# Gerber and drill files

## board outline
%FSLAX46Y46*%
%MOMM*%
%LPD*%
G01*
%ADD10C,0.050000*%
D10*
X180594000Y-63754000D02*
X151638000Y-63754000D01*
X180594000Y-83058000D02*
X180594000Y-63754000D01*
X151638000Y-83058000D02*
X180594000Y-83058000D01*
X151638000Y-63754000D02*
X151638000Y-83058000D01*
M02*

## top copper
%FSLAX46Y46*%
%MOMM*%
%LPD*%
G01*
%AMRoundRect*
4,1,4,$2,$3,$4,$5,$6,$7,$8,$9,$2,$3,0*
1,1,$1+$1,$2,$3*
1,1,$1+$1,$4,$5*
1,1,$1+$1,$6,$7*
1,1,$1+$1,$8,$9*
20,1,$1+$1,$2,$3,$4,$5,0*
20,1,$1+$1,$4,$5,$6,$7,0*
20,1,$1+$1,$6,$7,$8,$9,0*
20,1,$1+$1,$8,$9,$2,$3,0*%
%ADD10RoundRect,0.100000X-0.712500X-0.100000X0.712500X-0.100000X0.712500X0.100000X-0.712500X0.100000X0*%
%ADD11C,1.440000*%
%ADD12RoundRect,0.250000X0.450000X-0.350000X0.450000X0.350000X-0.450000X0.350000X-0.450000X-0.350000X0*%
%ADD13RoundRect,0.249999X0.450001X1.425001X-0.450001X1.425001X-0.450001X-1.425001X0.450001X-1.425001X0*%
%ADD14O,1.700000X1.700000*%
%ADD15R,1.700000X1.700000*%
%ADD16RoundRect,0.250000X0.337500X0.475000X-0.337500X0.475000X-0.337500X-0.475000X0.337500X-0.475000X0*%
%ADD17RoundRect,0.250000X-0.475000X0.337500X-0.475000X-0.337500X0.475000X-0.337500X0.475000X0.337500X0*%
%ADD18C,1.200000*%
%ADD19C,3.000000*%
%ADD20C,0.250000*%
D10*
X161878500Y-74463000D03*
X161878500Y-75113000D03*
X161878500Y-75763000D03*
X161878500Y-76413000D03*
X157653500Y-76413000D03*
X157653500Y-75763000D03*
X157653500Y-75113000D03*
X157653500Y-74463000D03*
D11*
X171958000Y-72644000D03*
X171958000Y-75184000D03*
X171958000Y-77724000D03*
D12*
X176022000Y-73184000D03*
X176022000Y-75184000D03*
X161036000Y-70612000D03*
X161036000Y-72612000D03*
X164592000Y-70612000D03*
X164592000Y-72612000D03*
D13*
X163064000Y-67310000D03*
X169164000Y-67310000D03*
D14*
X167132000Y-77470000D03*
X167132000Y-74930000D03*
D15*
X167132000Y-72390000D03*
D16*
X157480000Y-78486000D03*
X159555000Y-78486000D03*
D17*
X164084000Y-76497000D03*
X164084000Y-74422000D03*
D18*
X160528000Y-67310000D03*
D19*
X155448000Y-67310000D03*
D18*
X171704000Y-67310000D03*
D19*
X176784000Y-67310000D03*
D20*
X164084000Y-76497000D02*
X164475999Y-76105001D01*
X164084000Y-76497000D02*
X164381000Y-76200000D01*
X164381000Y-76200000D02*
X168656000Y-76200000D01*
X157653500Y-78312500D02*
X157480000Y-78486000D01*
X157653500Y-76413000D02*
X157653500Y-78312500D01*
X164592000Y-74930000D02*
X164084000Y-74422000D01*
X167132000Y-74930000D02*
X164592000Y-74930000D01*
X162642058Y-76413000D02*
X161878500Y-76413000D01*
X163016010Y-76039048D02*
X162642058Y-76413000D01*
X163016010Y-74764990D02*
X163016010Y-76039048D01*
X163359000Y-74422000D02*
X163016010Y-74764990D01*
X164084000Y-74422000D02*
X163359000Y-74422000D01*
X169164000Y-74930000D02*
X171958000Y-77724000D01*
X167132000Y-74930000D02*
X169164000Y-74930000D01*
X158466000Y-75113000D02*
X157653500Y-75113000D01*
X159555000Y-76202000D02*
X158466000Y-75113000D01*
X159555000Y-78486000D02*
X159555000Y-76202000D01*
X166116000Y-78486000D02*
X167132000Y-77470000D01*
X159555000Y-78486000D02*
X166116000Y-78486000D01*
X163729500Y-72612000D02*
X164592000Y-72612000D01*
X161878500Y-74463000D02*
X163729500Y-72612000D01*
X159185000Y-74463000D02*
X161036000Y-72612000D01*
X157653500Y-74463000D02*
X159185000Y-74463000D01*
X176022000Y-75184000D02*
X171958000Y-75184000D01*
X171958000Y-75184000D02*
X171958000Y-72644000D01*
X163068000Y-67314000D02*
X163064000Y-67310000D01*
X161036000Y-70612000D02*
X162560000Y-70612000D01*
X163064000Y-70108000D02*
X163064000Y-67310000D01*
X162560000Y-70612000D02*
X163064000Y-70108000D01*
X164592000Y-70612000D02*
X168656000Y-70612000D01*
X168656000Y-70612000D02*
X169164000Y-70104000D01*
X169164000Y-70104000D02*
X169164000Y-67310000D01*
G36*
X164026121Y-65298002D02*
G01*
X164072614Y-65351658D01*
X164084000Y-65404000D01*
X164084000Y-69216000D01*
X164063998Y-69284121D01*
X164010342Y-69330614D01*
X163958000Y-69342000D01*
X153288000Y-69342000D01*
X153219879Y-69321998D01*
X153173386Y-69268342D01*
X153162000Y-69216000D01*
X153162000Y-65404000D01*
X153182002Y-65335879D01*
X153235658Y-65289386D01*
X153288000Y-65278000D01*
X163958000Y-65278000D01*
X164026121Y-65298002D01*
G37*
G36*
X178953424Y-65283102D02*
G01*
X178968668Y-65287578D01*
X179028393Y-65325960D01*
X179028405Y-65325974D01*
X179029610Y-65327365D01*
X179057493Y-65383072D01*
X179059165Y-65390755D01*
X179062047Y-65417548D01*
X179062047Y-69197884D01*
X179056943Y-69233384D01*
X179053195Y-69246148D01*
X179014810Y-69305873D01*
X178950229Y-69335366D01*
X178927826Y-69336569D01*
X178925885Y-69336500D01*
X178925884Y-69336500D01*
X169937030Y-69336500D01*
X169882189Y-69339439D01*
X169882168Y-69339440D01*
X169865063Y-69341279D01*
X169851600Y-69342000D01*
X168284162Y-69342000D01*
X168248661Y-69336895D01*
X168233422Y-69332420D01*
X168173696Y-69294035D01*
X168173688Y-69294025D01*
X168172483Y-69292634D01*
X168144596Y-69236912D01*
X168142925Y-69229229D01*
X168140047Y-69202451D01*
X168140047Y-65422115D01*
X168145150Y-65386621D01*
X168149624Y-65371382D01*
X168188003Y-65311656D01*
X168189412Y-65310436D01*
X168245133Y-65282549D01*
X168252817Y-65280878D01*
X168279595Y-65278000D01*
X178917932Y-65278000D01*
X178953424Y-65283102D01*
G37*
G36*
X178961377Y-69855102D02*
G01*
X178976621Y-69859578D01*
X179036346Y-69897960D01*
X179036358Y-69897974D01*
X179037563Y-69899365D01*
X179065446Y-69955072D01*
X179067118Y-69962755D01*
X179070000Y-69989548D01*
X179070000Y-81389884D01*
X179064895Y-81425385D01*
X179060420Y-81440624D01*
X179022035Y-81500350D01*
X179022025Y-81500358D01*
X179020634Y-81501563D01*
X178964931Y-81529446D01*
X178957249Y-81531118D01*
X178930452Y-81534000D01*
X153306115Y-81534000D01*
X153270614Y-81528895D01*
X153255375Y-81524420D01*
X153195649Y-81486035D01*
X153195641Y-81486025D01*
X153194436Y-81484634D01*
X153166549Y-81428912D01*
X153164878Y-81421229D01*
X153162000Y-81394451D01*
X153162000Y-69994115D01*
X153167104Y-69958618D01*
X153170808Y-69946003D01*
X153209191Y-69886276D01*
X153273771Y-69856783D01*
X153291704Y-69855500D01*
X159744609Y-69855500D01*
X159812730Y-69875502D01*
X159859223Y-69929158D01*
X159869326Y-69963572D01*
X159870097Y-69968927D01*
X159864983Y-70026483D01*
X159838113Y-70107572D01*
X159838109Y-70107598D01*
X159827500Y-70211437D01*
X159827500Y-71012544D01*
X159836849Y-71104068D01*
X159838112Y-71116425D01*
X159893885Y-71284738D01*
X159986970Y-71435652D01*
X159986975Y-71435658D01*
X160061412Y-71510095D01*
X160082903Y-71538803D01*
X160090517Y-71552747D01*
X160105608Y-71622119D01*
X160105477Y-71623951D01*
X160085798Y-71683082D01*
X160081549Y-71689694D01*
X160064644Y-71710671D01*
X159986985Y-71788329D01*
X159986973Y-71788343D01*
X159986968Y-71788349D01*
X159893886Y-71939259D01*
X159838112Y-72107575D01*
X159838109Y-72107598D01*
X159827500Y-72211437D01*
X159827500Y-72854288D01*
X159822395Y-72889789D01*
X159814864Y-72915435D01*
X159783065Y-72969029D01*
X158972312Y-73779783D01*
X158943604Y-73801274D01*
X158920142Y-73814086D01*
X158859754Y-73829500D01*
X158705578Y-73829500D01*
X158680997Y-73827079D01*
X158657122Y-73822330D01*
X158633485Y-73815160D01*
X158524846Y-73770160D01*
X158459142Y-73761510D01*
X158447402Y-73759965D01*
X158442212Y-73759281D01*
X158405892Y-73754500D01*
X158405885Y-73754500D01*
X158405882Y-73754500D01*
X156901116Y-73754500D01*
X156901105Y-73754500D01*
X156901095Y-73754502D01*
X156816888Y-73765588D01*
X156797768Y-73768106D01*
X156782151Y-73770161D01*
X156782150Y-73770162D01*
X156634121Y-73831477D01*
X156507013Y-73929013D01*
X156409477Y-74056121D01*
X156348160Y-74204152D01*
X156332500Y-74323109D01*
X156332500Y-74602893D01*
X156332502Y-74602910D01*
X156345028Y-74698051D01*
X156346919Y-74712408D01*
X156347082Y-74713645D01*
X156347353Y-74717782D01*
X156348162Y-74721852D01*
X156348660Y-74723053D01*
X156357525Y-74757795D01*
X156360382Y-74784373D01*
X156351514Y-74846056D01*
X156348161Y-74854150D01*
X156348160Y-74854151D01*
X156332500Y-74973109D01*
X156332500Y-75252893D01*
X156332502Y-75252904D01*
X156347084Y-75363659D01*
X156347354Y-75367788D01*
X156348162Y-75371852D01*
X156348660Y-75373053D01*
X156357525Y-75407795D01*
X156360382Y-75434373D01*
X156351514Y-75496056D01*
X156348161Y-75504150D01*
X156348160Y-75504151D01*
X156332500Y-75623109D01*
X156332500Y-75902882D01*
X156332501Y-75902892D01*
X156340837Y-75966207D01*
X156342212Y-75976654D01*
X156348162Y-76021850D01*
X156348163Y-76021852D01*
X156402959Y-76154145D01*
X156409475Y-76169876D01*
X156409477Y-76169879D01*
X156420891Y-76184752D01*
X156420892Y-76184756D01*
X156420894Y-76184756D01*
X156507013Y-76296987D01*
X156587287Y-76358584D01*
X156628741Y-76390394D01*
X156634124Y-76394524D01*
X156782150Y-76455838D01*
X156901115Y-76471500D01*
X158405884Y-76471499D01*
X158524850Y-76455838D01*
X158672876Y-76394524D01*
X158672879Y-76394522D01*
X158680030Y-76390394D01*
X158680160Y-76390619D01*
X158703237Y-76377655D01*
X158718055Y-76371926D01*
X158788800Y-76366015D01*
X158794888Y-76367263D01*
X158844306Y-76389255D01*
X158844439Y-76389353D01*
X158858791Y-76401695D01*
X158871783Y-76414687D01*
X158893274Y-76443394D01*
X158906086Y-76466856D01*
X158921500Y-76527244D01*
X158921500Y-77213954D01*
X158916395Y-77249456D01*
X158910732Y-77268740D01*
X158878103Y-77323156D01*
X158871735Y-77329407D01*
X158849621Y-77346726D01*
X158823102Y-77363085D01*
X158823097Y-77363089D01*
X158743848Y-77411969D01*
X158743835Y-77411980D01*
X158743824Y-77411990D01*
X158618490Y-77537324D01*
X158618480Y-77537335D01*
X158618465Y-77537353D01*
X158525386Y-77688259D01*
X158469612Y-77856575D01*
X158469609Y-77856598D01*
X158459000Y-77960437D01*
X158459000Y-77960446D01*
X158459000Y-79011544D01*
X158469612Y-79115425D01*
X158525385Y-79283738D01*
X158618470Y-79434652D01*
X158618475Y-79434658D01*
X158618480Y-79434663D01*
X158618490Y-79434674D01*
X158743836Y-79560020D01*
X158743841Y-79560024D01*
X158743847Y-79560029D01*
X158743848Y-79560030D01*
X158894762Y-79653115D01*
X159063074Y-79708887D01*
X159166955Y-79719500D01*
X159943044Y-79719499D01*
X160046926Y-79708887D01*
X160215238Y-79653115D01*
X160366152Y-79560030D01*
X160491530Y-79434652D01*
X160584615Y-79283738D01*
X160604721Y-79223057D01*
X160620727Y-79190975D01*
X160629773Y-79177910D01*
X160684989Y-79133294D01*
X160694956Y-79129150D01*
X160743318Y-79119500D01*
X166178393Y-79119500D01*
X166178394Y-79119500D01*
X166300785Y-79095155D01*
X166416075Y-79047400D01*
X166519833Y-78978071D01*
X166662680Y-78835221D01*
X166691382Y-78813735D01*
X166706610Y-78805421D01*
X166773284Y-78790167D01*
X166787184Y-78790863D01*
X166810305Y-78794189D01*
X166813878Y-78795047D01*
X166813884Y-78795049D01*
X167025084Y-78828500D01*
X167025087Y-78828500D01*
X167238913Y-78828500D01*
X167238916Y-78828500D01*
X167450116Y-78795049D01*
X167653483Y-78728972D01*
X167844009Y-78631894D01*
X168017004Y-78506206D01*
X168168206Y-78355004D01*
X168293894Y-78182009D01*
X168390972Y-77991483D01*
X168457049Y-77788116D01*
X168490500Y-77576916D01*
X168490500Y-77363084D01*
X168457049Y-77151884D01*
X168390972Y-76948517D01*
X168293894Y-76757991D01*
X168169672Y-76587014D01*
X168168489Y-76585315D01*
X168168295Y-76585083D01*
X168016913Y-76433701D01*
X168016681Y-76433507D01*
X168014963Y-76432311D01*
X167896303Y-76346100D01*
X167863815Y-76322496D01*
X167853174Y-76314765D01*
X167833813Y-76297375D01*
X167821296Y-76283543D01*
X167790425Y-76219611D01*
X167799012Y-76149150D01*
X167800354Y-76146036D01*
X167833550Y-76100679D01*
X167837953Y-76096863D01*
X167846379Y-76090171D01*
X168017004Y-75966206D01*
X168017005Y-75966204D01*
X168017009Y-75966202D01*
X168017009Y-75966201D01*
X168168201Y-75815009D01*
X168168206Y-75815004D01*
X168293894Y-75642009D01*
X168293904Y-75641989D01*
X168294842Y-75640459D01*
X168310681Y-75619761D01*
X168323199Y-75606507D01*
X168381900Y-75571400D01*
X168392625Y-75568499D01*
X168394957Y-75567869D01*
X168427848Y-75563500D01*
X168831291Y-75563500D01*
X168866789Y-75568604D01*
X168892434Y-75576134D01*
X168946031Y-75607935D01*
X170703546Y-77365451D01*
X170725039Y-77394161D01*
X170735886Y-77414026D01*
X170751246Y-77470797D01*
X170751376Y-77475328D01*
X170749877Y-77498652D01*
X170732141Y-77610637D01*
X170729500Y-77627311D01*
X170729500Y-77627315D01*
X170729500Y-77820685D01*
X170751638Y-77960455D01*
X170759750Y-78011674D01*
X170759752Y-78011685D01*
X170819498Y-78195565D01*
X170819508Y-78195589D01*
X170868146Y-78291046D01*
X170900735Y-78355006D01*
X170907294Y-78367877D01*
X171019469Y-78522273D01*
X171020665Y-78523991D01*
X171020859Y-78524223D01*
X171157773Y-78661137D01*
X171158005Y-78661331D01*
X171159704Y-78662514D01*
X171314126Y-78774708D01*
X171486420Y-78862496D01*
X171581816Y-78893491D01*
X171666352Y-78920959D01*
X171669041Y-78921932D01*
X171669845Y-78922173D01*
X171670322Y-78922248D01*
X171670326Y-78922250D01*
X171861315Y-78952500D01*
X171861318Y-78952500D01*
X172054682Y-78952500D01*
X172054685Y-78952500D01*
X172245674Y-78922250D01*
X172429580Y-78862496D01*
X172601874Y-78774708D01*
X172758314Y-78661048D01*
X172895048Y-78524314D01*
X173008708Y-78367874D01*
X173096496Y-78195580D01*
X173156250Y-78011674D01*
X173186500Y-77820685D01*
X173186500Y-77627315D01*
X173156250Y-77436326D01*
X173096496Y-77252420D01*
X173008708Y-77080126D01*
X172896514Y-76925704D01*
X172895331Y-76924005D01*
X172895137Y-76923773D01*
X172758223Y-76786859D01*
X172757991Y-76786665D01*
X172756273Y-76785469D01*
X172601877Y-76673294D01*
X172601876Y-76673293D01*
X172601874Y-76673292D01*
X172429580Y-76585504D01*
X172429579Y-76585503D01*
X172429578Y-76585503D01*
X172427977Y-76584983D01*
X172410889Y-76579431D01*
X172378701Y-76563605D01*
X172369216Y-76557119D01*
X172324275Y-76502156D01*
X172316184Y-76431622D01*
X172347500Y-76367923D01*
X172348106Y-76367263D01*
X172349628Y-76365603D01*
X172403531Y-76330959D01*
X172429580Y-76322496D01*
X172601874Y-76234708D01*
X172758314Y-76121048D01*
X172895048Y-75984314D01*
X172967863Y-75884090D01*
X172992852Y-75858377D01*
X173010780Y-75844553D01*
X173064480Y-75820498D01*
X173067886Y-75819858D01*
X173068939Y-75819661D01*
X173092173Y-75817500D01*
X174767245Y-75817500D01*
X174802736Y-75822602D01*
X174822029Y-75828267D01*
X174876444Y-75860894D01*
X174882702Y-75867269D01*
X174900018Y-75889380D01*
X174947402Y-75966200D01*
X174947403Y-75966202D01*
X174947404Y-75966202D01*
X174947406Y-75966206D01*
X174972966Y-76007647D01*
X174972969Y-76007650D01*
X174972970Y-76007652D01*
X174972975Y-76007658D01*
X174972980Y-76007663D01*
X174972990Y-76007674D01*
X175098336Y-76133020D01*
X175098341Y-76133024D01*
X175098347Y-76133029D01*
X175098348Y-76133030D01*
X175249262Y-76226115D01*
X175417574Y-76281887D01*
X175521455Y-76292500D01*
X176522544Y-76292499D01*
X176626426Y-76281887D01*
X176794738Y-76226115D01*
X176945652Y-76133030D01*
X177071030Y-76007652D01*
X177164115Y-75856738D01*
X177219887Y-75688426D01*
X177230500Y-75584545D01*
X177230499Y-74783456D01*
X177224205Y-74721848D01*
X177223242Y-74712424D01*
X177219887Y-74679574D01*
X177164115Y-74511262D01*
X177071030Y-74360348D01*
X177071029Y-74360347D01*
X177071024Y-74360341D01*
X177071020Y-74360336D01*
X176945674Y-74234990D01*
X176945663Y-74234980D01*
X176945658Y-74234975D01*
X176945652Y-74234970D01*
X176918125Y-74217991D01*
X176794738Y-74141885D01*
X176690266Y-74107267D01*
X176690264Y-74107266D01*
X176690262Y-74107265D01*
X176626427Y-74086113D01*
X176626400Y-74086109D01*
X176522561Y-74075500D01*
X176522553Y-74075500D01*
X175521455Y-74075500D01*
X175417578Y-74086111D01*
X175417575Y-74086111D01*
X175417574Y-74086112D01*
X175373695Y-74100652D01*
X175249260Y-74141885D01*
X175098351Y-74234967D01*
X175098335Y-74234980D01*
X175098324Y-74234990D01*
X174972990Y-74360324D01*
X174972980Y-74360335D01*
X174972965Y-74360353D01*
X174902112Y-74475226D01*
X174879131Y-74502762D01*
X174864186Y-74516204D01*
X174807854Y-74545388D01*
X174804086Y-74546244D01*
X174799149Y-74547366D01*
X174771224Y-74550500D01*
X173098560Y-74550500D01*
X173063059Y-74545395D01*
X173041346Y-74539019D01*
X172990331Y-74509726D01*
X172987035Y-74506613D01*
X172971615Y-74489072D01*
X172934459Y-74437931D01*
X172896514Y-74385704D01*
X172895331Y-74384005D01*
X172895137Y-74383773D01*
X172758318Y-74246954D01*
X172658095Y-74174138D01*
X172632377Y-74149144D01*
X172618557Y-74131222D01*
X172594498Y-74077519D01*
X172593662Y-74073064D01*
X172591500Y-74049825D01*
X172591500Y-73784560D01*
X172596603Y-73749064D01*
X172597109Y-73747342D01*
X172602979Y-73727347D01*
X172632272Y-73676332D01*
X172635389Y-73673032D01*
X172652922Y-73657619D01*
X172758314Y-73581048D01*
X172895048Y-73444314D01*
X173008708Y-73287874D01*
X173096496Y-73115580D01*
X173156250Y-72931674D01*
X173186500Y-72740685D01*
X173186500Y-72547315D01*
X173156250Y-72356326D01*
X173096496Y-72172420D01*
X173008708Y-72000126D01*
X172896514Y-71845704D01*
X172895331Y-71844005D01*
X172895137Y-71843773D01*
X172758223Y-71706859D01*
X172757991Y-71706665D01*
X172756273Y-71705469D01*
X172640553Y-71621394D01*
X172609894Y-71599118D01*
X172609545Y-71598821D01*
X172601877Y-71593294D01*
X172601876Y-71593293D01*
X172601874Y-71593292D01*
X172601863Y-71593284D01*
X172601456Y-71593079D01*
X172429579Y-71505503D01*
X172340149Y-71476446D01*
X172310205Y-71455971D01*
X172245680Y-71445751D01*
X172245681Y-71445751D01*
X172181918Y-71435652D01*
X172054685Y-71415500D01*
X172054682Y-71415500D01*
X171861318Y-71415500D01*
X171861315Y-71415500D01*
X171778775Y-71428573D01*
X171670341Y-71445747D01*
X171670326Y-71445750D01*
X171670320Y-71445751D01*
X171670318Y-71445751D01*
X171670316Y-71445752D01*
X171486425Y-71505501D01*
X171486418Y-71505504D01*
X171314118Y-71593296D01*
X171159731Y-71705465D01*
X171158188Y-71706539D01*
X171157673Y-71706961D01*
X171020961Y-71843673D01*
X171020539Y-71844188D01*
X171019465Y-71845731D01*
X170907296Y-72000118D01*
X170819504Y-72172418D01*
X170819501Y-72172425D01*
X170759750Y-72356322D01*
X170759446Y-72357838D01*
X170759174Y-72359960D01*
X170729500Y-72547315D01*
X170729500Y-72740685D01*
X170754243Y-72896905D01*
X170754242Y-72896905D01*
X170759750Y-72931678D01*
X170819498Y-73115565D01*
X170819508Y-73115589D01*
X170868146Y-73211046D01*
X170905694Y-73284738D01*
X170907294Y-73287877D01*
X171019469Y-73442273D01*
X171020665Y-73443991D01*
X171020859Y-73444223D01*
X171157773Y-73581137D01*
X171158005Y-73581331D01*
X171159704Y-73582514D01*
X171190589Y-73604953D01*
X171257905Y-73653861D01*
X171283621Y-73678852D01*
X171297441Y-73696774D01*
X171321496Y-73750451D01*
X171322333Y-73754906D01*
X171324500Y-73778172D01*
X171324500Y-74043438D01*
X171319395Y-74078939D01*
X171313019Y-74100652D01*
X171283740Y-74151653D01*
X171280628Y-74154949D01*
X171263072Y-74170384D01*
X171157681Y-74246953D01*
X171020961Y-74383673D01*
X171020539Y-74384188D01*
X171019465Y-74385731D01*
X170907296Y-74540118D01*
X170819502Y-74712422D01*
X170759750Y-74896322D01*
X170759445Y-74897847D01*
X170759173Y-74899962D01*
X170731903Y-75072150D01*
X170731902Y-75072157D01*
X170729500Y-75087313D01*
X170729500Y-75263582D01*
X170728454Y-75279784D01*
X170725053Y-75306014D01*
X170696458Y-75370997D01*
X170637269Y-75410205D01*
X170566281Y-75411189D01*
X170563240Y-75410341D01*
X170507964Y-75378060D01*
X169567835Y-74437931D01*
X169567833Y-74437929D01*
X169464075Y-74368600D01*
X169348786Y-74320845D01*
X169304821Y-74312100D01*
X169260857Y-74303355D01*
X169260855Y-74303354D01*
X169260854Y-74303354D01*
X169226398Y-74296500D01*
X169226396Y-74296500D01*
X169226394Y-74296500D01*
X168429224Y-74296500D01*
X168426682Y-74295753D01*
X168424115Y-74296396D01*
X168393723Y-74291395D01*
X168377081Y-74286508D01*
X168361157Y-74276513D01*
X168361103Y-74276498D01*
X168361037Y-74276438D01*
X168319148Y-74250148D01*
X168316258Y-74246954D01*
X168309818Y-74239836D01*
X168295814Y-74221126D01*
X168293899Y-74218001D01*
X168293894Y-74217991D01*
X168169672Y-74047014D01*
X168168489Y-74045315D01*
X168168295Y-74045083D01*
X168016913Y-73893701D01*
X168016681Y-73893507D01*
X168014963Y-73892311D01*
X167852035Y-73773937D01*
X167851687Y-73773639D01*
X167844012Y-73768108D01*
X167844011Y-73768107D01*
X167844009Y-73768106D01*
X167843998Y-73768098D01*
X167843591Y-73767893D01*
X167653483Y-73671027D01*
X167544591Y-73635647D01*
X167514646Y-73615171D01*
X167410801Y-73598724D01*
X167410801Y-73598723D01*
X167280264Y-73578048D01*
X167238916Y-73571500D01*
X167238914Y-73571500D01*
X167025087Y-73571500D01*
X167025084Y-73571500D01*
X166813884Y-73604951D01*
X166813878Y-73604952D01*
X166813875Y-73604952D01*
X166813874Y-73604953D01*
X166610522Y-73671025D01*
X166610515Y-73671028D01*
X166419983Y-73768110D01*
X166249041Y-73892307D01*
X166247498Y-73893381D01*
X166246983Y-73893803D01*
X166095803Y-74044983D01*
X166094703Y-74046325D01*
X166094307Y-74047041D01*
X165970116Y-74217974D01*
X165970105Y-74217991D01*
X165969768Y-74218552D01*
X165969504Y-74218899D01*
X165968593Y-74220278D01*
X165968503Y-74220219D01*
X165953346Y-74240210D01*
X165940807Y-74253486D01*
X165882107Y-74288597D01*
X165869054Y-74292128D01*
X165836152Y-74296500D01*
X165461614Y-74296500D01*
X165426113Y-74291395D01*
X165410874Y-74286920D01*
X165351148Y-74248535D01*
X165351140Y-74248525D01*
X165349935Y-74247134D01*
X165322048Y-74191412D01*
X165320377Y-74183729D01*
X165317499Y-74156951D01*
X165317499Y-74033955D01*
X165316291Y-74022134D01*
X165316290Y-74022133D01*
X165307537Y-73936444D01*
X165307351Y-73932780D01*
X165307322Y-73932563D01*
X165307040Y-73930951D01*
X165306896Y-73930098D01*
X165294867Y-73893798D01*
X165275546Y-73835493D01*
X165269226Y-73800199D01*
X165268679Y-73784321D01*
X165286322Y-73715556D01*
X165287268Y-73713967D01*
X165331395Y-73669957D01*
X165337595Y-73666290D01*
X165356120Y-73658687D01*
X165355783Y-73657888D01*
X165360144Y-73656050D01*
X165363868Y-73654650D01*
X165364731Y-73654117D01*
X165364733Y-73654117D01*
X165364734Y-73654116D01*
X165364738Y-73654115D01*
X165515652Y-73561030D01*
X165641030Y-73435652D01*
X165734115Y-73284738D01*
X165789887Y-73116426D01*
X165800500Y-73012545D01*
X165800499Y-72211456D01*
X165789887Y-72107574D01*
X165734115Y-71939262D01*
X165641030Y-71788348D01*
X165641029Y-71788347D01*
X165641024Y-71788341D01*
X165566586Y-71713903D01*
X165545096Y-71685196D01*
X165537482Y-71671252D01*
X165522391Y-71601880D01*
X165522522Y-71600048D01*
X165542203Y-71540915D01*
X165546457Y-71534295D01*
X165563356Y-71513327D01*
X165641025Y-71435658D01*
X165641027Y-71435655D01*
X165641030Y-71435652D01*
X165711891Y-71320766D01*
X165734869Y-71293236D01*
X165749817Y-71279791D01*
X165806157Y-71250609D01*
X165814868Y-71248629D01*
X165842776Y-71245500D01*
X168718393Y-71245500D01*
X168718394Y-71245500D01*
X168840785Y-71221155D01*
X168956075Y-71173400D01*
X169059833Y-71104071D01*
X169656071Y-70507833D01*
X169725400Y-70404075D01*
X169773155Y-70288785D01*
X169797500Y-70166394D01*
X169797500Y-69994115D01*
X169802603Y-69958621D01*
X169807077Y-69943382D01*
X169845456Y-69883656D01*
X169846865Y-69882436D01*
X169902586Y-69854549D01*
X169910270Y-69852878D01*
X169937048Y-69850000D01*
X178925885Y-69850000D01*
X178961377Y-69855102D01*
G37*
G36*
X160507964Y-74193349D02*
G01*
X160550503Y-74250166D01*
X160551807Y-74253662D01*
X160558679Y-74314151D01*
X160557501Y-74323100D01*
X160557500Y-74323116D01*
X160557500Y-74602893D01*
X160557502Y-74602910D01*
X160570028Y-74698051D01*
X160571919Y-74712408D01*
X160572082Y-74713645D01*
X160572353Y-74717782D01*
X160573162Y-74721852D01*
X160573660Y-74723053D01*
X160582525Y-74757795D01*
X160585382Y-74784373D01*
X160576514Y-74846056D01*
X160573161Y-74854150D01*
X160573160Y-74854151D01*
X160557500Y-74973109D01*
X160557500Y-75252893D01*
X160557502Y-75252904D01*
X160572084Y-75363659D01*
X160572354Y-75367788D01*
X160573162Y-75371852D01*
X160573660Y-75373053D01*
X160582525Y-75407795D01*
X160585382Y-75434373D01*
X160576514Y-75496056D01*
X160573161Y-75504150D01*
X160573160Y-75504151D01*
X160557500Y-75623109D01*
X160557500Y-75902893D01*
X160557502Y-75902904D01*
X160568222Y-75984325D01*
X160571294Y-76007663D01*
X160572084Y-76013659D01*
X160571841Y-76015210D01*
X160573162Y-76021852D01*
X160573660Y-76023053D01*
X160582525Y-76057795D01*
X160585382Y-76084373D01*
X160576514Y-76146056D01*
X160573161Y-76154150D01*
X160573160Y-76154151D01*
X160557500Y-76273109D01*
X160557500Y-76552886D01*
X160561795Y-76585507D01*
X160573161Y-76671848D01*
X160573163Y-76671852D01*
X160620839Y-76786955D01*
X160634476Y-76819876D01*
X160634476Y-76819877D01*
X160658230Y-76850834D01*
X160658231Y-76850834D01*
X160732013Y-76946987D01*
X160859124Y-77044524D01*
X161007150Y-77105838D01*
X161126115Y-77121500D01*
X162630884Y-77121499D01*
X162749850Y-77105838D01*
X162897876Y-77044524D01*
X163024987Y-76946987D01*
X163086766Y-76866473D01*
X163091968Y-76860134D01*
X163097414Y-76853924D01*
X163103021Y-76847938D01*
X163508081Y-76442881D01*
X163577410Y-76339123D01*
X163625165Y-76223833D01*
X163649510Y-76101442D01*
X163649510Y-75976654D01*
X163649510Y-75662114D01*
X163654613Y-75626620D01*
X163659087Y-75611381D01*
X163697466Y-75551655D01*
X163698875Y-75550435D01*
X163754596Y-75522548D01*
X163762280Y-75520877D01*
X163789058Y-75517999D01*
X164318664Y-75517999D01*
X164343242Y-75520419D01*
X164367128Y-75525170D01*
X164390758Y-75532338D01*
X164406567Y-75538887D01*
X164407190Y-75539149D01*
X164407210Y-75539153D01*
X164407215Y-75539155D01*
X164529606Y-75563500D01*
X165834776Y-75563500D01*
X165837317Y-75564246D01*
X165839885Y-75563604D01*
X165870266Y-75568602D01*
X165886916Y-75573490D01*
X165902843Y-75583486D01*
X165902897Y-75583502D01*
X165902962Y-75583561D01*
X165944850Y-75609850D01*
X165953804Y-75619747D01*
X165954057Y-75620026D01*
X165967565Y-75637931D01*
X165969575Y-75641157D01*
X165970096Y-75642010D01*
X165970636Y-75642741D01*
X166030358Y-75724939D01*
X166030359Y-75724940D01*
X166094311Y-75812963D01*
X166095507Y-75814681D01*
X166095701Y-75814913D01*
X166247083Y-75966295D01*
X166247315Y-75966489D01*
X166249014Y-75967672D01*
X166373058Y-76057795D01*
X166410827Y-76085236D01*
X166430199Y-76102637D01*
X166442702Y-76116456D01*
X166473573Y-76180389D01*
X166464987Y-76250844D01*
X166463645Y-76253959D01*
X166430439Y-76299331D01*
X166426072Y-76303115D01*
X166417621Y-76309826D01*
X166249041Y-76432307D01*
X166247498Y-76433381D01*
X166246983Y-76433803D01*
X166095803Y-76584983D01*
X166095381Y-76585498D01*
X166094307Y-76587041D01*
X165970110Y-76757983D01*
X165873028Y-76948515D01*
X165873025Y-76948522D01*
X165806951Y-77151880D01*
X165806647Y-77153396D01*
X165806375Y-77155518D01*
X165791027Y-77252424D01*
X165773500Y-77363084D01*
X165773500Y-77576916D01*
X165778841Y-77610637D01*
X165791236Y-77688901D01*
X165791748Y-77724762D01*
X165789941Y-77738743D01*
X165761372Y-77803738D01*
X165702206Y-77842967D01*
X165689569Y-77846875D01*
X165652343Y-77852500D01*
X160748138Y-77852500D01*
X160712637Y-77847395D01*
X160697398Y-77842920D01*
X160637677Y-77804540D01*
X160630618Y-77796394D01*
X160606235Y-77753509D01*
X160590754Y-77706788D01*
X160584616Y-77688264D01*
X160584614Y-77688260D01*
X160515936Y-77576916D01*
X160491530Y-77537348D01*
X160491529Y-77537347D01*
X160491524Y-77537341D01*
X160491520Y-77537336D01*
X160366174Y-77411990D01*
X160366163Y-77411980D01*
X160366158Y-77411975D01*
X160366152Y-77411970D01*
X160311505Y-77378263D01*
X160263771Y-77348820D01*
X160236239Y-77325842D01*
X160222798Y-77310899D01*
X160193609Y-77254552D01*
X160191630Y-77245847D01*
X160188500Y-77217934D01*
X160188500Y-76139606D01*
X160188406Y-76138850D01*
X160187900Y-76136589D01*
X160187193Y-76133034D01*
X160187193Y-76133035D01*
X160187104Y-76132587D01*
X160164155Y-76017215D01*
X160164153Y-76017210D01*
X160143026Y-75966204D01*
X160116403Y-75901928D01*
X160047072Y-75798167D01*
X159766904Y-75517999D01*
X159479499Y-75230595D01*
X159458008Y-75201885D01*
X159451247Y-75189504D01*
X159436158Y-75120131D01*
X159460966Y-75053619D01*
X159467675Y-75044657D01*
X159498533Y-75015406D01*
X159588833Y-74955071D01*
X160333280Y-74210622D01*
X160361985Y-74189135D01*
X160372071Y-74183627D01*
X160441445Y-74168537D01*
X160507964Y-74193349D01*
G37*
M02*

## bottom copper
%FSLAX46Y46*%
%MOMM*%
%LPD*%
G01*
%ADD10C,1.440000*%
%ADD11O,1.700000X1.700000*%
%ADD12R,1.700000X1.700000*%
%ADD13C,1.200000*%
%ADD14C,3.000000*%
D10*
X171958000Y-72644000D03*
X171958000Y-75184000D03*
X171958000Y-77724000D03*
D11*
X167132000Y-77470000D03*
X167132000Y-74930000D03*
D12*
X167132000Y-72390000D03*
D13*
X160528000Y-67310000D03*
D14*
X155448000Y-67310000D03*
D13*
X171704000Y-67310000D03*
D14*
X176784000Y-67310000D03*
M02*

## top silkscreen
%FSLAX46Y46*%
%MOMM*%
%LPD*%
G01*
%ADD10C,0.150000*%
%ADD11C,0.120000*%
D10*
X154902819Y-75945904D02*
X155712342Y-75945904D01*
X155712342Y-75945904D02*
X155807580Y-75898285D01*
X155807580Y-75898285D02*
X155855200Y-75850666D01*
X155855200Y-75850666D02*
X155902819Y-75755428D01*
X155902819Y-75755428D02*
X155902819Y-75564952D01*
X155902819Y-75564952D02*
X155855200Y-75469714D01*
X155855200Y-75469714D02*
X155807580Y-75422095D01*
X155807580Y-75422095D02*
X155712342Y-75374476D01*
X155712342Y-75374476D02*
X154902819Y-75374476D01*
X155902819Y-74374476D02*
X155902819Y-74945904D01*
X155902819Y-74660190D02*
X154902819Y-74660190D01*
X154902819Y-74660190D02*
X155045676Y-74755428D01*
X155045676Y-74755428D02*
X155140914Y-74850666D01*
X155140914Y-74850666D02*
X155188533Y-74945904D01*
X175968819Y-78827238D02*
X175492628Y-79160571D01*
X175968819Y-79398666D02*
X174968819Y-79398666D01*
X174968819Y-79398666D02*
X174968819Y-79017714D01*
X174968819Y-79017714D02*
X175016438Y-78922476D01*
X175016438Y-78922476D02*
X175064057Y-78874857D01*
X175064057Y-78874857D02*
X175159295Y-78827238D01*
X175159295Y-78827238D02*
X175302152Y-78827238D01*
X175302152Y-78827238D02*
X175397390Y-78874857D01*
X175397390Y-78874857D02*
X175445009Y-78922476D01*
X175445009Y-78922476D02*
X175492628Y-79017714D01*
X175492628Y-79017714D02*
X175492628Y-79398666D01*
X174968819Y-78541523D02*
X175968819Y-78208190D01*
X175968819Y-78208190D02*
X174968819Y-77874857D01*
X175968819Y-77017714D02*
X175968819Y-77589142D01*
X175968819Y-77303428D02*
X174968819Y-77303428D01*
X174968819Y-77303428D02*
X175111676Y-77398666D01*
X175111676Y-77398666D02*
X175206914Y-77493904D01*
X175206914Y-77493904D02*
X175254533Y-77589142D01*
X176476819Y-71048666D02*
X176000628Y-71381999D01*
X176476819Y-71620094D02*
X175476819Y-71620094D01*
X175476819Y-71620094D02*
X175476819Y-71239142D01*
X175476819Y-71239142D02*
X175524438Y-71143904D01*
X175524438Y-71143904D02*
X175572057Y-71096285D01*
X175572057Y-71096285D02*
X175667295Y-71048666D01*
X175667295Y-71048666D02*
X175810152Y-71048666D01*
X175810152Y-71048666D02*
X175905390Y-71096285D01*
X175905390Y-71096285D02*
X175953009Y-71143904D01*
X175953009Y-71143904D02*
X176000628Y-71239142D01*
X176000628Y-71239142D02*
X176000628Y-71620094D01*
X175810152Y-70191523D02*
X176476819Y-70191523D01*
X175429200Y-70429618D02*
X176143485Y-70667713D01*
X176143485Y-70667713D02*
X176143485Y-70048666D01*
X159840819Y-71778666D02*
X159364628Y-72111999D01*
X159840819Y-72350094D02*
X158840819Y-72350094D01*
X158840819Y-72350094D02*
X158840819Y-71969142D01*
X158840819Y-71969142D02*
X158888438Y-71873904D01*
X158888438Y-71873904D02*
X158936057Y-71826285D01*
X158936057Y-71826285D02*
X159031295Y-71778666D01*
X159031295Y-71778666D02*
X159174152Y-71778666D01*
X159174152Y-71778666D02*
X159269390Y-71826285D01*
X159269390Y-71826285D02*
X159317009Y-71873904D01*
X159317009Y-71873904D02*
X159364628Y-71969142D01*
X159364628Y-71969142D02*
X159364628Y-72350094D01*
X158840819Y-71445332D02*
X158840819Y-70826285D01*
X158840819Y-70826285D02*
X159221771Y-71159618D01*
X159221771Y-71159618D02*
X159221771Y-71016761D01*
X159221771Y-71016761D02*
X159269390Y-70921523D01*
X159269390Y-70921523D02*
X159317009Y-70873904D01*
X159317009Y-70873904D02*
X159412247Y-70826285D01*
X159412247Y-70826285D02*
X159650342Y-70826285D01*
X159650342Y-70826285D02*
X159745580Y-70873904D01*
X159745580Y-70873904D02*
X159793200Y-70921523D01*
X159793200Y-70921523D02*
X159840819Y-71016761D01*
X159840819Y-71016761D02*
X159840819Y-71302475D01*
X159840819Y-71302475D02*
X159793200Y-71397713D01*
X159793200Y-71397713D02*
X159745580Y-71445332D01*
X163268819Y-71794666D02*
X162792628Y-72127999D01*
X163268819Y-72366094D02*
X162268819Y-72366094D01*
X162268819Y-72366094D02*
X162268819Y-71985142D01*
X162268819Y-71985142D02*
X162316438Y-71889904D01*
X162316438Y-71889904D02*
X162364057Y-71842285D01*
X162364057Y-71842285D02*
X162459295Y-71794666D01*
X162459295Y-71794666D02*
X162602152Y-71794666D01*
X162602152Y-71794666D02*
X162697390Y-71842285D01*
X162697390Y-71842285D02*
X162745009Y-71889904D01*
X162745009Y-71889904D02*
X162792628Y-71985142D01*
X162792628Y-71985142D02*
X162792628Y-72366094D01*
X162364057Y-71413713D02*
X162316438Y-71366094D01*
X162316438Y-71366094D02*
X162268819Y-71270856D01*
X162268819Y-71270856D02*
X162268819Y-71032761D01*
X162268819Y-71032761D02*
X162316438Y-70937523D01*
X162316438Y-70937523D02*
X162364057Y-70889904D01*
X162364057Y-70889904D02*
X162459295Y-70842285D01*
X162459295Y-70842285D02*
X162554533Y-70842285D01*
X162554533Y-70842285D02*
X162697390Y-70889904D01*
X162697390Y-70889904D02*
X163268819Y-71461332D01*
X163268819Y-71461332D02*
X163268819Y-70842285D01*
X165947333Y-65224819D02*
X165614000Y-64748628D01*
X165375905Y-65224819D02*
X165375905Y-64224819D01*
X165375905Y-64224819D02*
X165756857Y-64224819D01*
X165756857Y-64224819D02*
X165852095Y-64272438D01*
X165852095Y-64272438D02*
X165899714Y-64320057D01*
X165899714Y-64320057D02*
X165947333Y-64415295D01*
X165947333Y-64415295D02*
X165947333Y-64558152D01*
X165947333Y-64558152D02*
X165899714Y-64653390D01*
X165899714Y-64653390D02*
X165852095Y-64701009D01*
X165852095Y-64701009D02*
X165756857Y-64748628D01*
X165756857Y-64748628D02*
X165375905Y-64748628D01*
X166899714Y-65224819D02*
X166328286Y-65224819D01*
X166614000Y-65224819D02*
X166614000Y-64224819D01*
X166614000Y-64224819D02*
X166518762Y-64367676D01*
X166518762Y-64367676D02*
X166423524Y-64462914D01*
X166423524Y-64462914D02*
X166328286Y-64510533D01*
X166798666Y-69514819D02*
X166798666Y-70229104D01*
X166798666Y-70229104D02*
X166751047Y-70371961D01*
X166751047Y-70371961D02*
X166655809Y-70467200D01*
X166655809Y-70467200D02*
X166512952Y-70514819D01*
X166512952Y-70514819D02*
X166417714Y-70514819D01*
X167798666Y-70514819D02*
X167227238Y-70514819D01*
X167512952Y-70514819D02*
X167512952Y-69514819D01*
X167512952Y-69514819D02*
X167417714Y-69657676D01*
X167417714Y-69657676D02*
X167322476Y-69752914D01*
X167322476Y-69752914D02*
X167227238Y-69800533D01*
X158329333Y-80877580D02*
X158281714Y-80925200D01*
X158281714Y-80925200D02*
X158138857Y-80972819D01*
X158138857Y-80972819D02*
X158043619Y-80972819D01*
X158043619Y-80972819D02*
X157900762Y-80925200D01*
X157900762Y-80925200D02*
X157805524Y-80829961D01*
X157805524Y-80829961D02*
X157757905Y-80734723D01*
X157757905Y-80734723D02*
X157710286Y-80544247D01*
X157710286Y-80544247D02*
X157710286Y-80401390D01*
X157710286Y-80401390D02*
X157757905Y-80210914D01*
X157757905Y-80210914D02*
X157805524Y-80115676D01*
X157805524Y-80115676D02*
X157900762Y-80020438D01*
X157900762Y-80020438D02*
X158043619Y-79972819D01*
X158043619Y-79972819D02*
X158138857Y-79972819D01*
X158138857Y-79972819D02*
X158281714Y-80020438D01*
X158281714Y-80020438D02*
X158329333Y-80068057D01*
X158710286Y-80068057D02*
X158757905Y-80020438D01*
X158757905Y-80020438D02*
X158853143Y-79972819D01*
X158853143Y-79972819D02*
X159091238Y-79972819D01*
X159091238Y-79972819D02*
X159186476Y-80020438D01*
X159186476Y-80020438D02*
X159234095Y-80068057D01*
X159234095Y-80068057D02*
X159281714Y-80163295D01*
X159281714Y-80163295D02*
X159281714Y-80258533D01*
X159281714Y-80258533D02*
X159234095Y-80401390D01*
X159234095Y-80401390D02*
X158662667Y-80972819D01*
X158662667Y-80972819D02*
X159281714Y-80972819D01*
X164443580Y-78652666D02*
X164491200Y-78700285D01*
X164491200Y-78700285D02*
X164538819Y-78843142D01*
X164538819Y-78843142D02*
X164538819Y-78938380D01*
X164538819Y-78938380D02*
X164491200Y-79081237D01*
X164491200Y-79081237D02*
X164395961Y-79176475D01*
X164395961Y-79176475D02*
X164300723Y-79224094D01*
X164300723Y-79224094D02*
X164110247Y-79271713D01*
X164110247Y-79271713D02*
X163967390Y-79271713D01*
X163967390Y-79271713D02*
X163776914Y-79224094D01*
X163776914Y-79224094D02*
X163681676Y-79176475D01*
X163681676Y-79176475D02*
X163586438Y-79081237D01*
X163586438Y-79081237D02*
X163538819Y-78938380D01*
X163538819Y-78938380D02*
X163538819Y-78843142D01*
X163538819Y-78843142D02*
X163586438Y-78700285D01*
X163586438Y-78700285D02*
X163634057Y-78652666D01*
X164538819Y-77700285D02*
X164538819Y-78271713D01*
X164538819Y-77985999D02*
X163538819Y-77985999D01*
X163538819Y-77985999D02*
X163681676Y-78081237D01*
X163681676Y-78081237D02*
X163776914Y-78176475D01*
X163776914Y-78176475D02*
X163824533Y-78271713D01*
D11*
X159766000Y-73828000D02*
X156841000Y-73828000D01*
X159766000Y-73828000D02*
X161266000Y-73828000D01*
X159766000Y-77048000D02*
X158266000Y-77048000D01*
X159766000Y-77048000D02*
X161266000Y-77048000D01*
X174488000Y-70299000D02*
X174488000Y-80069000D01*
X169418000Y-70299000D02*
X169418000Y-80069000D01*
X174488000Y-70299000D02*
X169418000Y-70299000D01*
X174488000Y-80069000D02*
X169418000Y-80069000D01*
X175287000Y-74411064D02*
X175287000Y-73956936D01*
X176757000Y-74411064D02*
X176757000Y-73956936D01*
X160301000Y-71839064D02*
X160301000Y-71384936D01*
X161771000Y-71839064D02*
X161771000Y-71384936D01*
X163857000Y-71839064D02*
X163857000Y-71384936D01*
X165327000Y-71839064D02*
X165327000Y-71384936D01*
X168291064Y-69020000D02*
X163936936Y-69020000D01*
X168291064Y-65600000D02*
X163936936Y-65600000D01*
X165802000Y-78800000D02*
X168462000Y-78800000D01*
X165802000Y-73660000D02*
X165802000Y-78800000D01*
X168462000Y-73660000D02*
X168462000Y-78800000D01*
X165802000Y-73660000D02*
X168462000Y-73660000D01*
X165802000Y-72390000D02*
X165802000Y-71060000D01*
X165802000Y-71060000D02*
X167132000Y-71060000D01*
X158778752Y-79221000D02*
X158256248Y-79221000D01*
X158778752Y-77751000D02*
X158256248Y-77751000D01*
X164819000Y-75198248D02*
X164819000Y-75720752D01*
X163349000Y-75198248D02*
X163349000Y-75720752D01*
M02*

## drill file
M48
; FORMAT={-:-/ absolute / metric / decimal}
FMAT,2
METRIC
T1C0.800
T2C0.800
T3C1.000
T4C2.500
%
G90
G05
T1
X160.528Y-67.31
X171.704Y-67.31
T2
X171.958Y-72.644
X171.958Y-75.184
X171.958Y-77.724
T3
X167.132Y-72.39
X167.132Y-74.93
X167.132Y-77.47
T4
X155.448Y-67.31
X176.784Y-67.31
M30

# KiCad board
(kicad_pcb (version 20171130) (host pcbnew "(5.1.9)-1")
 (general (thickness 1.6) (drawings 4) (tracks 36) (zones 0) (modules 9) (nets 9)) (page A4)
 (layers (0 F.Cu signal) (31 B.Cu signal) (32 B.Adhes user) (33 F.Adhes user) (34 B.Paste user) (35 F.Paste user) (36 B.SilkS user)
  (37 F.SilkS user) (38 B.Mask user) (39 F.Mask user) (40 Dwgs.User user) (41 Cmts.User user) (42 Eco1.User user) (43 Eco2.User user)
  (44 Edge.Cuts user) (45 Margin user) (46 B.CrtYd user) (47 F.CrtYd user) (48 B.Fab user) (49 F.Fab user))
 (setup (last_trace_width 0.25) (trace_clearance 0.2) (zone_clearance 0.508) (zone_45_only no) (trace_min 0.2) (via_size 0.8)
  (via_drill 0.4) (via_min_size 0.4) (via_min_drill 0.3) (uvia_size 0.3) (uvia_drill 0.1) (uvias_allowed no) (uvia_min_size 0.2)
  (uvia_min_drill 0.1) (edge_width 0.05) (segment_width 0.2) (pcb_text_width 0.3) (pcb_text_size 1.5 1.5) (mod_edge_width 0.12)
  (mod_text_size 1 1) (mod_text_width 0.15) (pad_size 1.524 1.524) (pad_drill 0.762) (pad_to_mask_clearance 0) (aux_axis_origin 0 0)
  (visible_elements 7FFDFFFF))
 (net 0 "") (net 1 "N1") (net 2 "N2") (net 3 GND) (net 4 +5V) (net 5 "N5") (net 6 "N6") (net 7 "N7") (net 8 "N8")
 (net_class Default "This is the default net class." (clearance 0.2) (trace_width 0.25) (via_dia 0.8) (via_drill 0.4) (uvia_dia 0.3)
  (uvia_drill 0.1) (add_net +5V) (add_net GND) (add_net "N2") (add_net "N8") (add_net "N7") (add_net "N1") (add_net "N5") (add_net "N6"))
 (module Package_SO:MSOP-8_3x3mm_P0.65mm (layer F.Cu) (at 159.766 75.438)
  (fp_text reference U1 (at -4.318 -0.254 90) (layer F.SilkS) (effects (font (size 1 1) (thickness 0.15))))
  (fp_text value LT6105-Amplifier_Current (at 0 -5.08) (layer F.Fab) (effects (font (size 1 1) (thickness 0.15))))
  (fp_line (start 0 -1.61) (end -2.925 -1.61) (layer F.SilkS) (width 0.12))
  (fp_line (start 0 -1.61) (end 1.5 -1.61) (layer F.SilkS) (width 0.12))
  (fp_line (start 0 1.61) (end -1.5 1.61) (layer F.SilkS) (width 0.12))
  (fp_line (start 0 1.61) (end 1.5 1.61) (layer F.SilkS) (width 0.12))
  (pad 8 smd roundrect (at 2.1125 -0.975) (size 1.625 0.4) (layers F.Cu F.Paste F.Mask) (roundrect_rratio 0.25) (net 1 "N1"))
  (pad 7 smd roundrect (at 2.1125 -0.325) (size 1.625 0.4) (layers F.Cu F.Paste F.Mask) (roundrect_rratio 0.25))
  (pad 6 smd roundrect (at 2.1125 0.325) (size 1.625 0.4) (layers F.Cu F.Paste F.Mask) (roundrect_rratio 0.25))
  (pad 5 smd roundrect (at 2.1125 0.975) (size 1.625 0.4) (layers F.Cu F.Paste F.Mask) (roundrect_rratio 0.25) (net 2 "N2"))
  (pad 4 smd roundrect (at -2.1125 0.975) (size 1.625 0.4) (layers F.Cu F.Paste F.Mask) (roundrect_rratio 0.25) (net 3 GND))
  (pad 3 smd roundrect (at -2.1125 0.325) (size 1.625 0.4) (layers F.Cu F.Paste F.Mask) (roundrect_rratio 0.25))
  (pad 2 smd roundrect (at -2.1125 -0.325) (size 1.625 0.4) (layers F.Cu F.Paste F.Mask) (roundrect_rratio 0.25) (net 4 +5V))
  (pad 1 smd roundrect (at -2.1125 -0.975) (size 1.625 0.4) (layers F.Cu F.Paste F.Mask) (roundrect_rratio 0.25) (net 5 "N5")))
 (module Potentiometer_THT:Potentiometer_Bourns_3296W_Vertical (layer F.Cu) (at 171.958 77.724 270)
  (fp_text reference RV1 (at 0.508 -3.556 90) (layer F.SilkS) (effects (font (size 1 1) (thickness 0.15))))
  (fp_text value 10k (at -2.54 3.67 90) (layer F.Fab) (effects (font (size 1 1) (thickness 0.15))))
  (fp_line (start -7.425 -2.53) (end 2.345 -2.53) (layer F.SilkS) (width 0.12))
  (fp_line (start -7.425 2.54) (end 2.345 2.54) (layer F.SilkS) (width 0.12))
  (fp_line (start -7.425 -2.53) (end -7.425 2.54) (layer F.SilkS) (width 0.12))
  (fp_line (start 2.345 -2.53) (end 2.345 2.54) (layer F.SilkS) (width 0.12))
  (pad 3 thru_hole circle (at -5.08 0 270) (size 1.44 1.44) (drill 0.8) (layers *.Cu *.Mask) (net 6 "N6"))
  (pad 2 thru_hole circle (at -2.54 0 270) (size 1.44 1.44) (drill 0.8) (layers *.Cu *.Mask) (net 6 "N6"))
  (pad 1 thru_hole circle (at 0 0 270) (size 1.44 1.44) (drill 0.8) (layers *.Cu *.Mask) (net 2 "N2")))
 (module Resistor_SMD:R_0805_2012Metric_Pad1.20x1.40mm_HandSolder (layer F.Cu) (at 176.022 74.184 90)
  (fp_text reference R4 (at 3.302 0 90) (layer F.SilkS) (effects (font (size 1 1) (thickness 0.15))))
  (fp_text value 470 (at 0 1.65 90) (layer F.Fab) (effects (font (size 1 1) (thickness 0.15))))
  (fp_line (start -0.227064 -0.735) (end 0.227064 -0.735) (layer F.SilkS) (width 0.12))
  (fp_line (start -0.227064 0.735) (end 0.227064 0.735) (layer F.SilkS) (width 0.12))
  (pad 2 smd roundrect (at 1 0 90) (size 1.2 1.4) (layers F.Cu F.Paste F.Mask) (roundrect_rratio 0.208333) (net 3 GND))
  (pad 1 smd roundrect (at -1 0 90) (size 1.2 1.4) (layers F.Cu F.Paste F.Mask) (roundrect_rratio 0.208333) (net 6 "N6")))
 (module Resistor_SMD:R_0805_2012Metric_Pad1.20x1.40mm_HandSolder (layer F.Cu) (at 161.036 71.612 90)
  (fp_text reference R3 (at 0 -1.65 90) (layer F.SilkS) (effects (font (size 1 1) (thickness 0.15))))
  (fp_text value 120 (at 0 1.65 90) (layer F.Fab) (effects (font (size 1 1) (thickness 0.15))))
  (fp_line (start -0.227064 -0.735) (end 0.227064 -0.735) (layer F.SilkS) (width 0.12))
  (fp_line (start -0.227064 0.735) (end 0.227064 0.735) (layer F.SilkS) (width 0.12))
  (pad 2 smd roundrect (at 1 0 90) (size 1.2 1.4) (layers F.Cu F.Paste F.Mask) (roundrect_rratio 0.208333) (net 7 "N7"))
  (pad 1 smd roundrect (at -1 0 90) (size 1.2 1.4) (layers F.Cu F.Paste F.Mask) (roundrect_rratio 0.208333) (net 5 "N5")))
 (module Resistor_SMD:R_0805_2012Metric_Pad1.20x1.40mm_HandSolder (layer F.Cu) (at 164.592 71.612 90)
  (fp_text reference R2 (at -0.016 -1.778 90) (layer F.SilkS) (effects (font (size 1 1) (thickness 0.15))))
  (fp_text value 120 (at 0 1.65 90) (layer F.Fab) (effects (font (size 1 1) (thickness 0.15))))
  (fp_line (start -0.227064 -0.735) (end 0.227064 -0.735) (layer F.SilkS) (width 0.12))
  (fp_line (start -0.227064 0.735) (end 0.227064 0.735) (layer F.SilkS) (width 0.12))
  (pad 2 smd roundrect (at 1 0 90) (size 1.2 1.4) (layers F.Cu F.Paste F.Mask) (roundrect_rratio 0.208333) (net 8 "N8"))
  (pad 1 smd roundrect (at -1 0 90) (size 1.2 1.4) (layers F.Cu F.Paste F.Mask) (roundrect_rratio 0.208333) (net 1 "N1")))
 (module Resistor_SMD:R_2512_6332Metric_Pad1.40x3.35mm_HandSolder (layer F.Cu) (at 166.114 67.31 180)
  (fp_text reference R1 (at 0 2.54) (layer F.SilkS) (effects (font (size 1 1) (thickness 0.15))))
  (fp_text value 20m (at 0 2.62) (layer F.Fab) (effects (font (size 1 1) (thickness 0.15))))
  (fp_line (start -2.177064 -1.71) (end 2.177064 -1.71) (layer F.SilkS) (width 0.12))
  (fp_line (start -2.177064 1.71) (end 2.177064 1.71) (layer F.SilkS) (width 0.12))
  (pad 2 smd roundrect (at 3.05 0 180) (size 1.4 3.35) (layers F.Cu F.Paste F.Mask) (roundrect_rratio 0.178571) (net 7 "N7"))
  (pad 1 smd roundrect (at -3.05 0 180) (size 1.4 3.35) (layers F.Cu F.Paste F.Mask) (roundrect_rratio 0.178571) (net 8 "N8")))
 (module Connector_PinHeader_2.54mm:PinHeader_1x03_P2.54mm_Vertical (layer F.Cu) (at 167.132 72.39)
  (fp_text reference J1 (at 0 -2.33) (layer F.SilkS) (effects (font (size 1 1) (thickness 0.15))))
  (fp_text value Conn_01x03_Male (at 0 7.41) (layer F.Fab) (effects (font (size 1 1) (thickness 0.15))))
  (fp_line (start -1.33 6.41) (end 1.33 6.41) (layer F.SilkS) (width 0.12))
  (fp_line (start -1.33 1.27) (end -1.33 6.41) (layer F.SilkS) (width 0.12))
  (fp_line (start 1.33 1.27) (end 1.33 6.41) (layer F.SilkS) (width 0.12))
  (fp_line (start -1.33 1.27) (end 1.33 1.27) (layer F.SilkS) (width 0.12))
  (fp_line (start -1.33 0) (end -1.33 -1.33) (layer F.SilkS) (width 0.12))
  (fp_line (start -1.33 -1.33) (end 0 -1.33) (layer F.SilkS) (width 0.12))
  (pad 3 thru_hole oval (at 0 5.08) (size 1.7 1.7) (drill 1) (layers *.Cu *.Mask) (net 4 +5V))
  (pad 2 thru_hole oval (at 0 2.54) (size 1.7 1.7) (drill 1) (layers *.Cu *.Mask) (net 2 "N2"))
  (pad 1 thru_hole rect (at 0 0) (size 1.7 1.7) (drill 1) (layers *.Cu *.Mask) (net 3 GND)))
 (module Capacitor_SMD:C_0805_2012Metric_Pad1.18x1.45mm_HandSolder (layer F.Cu) (at 158.5175 78.486 180)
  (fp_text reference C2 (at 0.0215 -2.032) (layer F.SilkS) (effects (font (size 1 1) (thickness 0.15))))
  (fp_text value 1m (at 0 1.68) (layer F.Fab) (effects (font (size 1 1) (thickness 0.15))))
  (fp_line (start -0.261252 -0.735) (end 0.261252 -0.735) (layer F.SilkS) (width 0.12))
  (fp_line (start -0.261252 0.735) (end 0.261252 0.735) (layer F.SilkS) (width 0.12))
  (pad 2 smd roundrect (at 1.0375 0 180) (size 1.175 1.45) (layers F.Cu F.Paste F.Mask) (roundrect_rratio 0.212766) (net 3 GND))
  (pad 1 smd roundrect (at -1.0375 0 180) (size 1.175 1.45) (layers F.Cu F.Paste F.Mask) (roundrect_rratio 0.212766) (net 4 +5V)))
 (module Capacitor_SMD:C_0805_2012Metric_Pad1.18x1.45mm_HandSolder (layer F.Cu) (at 164.084 75.4595 270)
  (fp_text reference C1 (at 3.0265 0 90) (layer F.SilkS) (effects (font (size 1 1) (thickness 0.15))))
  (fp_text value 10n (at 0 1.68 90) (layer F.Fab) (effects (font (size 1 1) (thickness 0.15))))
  (fp_line (start -0.261252 -0.735) (end 0.261252 -0.735) (layer F.SilkS) (width 0.12))
  (fp_line (start -0.261252 0.735) (end 0.261252 0.735) (layer F.SilkS) (width 0.12))
  (pad 2 smd roundrect (at 1.0375 0 270) (size 1.175 1.45) (layers F.Cu F.Paste F.Mask) (roundrect_rratio 0.212766) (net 3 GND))
  (pad 1 smd roundrect (at -1.0375 0 270) (size 1.175 1.45) (layers F.Cu F.Paste F.Mask) (roundrect_rratio 0.212766) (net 2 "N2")))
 (gr_line (start 180.594 63.754) (end 151.638 63.754) (layer Edge.Cuts) (width 0.05))
 (gr_line (start 180.594 83.058) (end 180.594 63.754) (layer Edge.Cuts) (width 0.05))
 (gr_line (start 151.638 83.058) (end 180.594 83.058) (layer Edge.Cuts) (width 0.05))
 (gr_line (start 151.638 63.754) (end 151.638 83.058) (layer Edge.Cuts) (width 0.05))
 (segment (start 164.084 76.497) (end 164.475999 76.105001) (width 0.25) (layer F.Cu) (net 3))
 (segment (start 164.084 76.497) (end 164.381 76.2) (width 0.25) (layer F.Cu) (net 3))
 (segment (start 164.381 76.2) (end 168.656 76.2) (width 0.25) (layer F.Cu) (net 3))
 (segment (start 157.6535 78.3125) (end 157.48 78.486) (width 0.25) (layer F.Cu) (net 3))
 (segment (start 157.6535 76.413) (end 157.6535 78.3125) (width 0.25) (layer F.Cu) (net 3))
 (segment (start 164.592 74.93) (end 164.084 74.422) (width 0.25) (layer F.Cu) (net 2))
 (segment (start 167.132 74.93) (end 164.592 74.93) (width 0.25) (layer F.Cu) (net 2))
 (segment (start 162.642058 76.413) (end 161.8785 76.413) (width 0.25) (layer F.Cu) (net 2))
 (segment (start 163.01601 76.039048) (end 162.642058 76.413) (width 0.25) (layer F.Cu) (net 2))
 (segment (start 163.01601 74.76499) (end 163.01601 76.039048) (width 0.25) (layer F.Cu) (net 2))
 (segment (start 163.359 74.422) (end 163.01601 74.76499) (width 0.25) (layer F.Cu) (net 2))
 (segment (start 164.084 74.422) (end 163.359 74.422) (width 0.25) (layer F.Cu) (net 2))
 (segment (start 169.164 74.93) (end 171.958 77.724) (width 0.25) (layer F.Cu) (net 2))
 (segment (start 167.132 74.93) (end 169.164 74.93) (width 0.25) (layer F.Cu) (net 2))
 (segment (start 158.466 75.113) (end 157.6535 75.113) (width 0.25) (layer F.Cu) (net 4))
 (segment (start 159.555 76.202) (end 158.466 75.113) (width 0.25) (layer F.Cu) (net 4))
 (segment (start 159.555 78.486) (end 159.555 76.202) (width 0.25) (layer F.Cu) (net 4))
 (segment (start 166.116 78.486) (end 167.132 77.47) (width 0.25) (layer F.Cu) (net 4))
 (segment (start 159.555 78.486) (end 166.116 78.486) (width 0.25) (layer F.Cu) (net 4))
 (segment (start 163.7295 72.612) (end 164.592 72.612) (width 0.25) (layer F.Cu) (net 1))
 (segment (start 161.8785 74.463) (end 163.7295 72.612) (width 0.25) (layer F.Cu) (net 1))
 (segment (start 159.185 74.463) (end 161.036 72.612) (width 0.25) (layer F.Cu) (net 5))
 (segment (start 157.6535 74.463) (end 159.185 74.463) (width 0.25) (layer F.Cu) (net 5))
 (segment (start 176.022 75.184) (end 171.958 75.184) (width 0.25) (layer F.Cu) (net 6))
 (segment (start 171.958 75.184) (end 171.958 72.644) (width 0.25) (layer F.Cu) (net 6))
 (via (at 160.528 67.31) (size 1.2) (drill 0.8) (layers F.Cu B.Cu) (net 7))
 (via (at 155.448 67.31) (size 3) (drill 2.5) (layers F.Cu B.Cu) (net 7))
 (segment (start 163.068 67.314) (end 163.064 67.31) (width 0.25) (layer F.Cu) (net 7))
 (segment (start 161.036 70.612) (end 162.56 70.612) (width 0.25) (layer F.Cu) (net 7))
 (segment (start 163.064 70.108) (end 163.064 67.31) (width 0.25) (layer F.Cu) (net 7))
 (segment (start 162.56 70.612) (end 163.064 70.108) (width 0.25) (layer F.Cu) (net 7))
 (via (at 171.704 67.31) (size 1.2) (drill 0.8) (layers F.Cu B.Cu) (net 8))
 (via (at 176.784 67.31) (size 3) (drill 2.5) (layers F.Cu B.Cu) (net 8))
 (segment (start 164.592 70.612) (end 168.656 70.612) (width 0.25) (layer F.Cu) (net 8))
 (segment (start 168.656 70.612) (end 169.164 70.104) (width 0.25) (layer F.Cu) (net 8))
 (segment (start 169.164 70.104) (end 169.164 67.31) (width 0.25) (layer F.Cu) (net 8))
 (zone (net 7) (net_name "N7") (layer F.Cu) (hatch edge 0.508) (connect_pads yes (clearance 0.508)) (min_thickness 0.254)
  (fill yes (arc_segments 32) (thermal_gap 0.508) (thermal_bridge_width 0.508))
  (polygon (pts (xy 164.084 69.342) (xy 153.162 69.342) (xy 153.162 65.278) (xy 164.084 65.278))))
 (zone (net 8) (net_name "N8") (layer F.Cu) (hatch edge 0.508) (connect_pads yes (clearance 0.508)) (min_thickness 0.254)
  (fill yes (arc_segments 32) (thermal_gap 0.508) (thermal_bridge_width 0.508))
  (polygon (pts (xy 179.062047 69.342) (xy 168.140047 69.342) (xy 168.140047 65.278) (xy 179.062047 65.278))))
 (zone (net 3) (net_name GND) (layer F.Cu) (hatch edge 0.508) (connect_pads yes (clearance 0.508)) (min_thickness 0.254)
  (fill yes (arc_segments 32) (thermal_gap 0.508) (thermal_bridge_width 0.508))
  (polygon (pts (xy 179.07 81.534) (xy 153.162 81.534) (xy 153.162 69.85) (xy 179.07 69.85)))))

